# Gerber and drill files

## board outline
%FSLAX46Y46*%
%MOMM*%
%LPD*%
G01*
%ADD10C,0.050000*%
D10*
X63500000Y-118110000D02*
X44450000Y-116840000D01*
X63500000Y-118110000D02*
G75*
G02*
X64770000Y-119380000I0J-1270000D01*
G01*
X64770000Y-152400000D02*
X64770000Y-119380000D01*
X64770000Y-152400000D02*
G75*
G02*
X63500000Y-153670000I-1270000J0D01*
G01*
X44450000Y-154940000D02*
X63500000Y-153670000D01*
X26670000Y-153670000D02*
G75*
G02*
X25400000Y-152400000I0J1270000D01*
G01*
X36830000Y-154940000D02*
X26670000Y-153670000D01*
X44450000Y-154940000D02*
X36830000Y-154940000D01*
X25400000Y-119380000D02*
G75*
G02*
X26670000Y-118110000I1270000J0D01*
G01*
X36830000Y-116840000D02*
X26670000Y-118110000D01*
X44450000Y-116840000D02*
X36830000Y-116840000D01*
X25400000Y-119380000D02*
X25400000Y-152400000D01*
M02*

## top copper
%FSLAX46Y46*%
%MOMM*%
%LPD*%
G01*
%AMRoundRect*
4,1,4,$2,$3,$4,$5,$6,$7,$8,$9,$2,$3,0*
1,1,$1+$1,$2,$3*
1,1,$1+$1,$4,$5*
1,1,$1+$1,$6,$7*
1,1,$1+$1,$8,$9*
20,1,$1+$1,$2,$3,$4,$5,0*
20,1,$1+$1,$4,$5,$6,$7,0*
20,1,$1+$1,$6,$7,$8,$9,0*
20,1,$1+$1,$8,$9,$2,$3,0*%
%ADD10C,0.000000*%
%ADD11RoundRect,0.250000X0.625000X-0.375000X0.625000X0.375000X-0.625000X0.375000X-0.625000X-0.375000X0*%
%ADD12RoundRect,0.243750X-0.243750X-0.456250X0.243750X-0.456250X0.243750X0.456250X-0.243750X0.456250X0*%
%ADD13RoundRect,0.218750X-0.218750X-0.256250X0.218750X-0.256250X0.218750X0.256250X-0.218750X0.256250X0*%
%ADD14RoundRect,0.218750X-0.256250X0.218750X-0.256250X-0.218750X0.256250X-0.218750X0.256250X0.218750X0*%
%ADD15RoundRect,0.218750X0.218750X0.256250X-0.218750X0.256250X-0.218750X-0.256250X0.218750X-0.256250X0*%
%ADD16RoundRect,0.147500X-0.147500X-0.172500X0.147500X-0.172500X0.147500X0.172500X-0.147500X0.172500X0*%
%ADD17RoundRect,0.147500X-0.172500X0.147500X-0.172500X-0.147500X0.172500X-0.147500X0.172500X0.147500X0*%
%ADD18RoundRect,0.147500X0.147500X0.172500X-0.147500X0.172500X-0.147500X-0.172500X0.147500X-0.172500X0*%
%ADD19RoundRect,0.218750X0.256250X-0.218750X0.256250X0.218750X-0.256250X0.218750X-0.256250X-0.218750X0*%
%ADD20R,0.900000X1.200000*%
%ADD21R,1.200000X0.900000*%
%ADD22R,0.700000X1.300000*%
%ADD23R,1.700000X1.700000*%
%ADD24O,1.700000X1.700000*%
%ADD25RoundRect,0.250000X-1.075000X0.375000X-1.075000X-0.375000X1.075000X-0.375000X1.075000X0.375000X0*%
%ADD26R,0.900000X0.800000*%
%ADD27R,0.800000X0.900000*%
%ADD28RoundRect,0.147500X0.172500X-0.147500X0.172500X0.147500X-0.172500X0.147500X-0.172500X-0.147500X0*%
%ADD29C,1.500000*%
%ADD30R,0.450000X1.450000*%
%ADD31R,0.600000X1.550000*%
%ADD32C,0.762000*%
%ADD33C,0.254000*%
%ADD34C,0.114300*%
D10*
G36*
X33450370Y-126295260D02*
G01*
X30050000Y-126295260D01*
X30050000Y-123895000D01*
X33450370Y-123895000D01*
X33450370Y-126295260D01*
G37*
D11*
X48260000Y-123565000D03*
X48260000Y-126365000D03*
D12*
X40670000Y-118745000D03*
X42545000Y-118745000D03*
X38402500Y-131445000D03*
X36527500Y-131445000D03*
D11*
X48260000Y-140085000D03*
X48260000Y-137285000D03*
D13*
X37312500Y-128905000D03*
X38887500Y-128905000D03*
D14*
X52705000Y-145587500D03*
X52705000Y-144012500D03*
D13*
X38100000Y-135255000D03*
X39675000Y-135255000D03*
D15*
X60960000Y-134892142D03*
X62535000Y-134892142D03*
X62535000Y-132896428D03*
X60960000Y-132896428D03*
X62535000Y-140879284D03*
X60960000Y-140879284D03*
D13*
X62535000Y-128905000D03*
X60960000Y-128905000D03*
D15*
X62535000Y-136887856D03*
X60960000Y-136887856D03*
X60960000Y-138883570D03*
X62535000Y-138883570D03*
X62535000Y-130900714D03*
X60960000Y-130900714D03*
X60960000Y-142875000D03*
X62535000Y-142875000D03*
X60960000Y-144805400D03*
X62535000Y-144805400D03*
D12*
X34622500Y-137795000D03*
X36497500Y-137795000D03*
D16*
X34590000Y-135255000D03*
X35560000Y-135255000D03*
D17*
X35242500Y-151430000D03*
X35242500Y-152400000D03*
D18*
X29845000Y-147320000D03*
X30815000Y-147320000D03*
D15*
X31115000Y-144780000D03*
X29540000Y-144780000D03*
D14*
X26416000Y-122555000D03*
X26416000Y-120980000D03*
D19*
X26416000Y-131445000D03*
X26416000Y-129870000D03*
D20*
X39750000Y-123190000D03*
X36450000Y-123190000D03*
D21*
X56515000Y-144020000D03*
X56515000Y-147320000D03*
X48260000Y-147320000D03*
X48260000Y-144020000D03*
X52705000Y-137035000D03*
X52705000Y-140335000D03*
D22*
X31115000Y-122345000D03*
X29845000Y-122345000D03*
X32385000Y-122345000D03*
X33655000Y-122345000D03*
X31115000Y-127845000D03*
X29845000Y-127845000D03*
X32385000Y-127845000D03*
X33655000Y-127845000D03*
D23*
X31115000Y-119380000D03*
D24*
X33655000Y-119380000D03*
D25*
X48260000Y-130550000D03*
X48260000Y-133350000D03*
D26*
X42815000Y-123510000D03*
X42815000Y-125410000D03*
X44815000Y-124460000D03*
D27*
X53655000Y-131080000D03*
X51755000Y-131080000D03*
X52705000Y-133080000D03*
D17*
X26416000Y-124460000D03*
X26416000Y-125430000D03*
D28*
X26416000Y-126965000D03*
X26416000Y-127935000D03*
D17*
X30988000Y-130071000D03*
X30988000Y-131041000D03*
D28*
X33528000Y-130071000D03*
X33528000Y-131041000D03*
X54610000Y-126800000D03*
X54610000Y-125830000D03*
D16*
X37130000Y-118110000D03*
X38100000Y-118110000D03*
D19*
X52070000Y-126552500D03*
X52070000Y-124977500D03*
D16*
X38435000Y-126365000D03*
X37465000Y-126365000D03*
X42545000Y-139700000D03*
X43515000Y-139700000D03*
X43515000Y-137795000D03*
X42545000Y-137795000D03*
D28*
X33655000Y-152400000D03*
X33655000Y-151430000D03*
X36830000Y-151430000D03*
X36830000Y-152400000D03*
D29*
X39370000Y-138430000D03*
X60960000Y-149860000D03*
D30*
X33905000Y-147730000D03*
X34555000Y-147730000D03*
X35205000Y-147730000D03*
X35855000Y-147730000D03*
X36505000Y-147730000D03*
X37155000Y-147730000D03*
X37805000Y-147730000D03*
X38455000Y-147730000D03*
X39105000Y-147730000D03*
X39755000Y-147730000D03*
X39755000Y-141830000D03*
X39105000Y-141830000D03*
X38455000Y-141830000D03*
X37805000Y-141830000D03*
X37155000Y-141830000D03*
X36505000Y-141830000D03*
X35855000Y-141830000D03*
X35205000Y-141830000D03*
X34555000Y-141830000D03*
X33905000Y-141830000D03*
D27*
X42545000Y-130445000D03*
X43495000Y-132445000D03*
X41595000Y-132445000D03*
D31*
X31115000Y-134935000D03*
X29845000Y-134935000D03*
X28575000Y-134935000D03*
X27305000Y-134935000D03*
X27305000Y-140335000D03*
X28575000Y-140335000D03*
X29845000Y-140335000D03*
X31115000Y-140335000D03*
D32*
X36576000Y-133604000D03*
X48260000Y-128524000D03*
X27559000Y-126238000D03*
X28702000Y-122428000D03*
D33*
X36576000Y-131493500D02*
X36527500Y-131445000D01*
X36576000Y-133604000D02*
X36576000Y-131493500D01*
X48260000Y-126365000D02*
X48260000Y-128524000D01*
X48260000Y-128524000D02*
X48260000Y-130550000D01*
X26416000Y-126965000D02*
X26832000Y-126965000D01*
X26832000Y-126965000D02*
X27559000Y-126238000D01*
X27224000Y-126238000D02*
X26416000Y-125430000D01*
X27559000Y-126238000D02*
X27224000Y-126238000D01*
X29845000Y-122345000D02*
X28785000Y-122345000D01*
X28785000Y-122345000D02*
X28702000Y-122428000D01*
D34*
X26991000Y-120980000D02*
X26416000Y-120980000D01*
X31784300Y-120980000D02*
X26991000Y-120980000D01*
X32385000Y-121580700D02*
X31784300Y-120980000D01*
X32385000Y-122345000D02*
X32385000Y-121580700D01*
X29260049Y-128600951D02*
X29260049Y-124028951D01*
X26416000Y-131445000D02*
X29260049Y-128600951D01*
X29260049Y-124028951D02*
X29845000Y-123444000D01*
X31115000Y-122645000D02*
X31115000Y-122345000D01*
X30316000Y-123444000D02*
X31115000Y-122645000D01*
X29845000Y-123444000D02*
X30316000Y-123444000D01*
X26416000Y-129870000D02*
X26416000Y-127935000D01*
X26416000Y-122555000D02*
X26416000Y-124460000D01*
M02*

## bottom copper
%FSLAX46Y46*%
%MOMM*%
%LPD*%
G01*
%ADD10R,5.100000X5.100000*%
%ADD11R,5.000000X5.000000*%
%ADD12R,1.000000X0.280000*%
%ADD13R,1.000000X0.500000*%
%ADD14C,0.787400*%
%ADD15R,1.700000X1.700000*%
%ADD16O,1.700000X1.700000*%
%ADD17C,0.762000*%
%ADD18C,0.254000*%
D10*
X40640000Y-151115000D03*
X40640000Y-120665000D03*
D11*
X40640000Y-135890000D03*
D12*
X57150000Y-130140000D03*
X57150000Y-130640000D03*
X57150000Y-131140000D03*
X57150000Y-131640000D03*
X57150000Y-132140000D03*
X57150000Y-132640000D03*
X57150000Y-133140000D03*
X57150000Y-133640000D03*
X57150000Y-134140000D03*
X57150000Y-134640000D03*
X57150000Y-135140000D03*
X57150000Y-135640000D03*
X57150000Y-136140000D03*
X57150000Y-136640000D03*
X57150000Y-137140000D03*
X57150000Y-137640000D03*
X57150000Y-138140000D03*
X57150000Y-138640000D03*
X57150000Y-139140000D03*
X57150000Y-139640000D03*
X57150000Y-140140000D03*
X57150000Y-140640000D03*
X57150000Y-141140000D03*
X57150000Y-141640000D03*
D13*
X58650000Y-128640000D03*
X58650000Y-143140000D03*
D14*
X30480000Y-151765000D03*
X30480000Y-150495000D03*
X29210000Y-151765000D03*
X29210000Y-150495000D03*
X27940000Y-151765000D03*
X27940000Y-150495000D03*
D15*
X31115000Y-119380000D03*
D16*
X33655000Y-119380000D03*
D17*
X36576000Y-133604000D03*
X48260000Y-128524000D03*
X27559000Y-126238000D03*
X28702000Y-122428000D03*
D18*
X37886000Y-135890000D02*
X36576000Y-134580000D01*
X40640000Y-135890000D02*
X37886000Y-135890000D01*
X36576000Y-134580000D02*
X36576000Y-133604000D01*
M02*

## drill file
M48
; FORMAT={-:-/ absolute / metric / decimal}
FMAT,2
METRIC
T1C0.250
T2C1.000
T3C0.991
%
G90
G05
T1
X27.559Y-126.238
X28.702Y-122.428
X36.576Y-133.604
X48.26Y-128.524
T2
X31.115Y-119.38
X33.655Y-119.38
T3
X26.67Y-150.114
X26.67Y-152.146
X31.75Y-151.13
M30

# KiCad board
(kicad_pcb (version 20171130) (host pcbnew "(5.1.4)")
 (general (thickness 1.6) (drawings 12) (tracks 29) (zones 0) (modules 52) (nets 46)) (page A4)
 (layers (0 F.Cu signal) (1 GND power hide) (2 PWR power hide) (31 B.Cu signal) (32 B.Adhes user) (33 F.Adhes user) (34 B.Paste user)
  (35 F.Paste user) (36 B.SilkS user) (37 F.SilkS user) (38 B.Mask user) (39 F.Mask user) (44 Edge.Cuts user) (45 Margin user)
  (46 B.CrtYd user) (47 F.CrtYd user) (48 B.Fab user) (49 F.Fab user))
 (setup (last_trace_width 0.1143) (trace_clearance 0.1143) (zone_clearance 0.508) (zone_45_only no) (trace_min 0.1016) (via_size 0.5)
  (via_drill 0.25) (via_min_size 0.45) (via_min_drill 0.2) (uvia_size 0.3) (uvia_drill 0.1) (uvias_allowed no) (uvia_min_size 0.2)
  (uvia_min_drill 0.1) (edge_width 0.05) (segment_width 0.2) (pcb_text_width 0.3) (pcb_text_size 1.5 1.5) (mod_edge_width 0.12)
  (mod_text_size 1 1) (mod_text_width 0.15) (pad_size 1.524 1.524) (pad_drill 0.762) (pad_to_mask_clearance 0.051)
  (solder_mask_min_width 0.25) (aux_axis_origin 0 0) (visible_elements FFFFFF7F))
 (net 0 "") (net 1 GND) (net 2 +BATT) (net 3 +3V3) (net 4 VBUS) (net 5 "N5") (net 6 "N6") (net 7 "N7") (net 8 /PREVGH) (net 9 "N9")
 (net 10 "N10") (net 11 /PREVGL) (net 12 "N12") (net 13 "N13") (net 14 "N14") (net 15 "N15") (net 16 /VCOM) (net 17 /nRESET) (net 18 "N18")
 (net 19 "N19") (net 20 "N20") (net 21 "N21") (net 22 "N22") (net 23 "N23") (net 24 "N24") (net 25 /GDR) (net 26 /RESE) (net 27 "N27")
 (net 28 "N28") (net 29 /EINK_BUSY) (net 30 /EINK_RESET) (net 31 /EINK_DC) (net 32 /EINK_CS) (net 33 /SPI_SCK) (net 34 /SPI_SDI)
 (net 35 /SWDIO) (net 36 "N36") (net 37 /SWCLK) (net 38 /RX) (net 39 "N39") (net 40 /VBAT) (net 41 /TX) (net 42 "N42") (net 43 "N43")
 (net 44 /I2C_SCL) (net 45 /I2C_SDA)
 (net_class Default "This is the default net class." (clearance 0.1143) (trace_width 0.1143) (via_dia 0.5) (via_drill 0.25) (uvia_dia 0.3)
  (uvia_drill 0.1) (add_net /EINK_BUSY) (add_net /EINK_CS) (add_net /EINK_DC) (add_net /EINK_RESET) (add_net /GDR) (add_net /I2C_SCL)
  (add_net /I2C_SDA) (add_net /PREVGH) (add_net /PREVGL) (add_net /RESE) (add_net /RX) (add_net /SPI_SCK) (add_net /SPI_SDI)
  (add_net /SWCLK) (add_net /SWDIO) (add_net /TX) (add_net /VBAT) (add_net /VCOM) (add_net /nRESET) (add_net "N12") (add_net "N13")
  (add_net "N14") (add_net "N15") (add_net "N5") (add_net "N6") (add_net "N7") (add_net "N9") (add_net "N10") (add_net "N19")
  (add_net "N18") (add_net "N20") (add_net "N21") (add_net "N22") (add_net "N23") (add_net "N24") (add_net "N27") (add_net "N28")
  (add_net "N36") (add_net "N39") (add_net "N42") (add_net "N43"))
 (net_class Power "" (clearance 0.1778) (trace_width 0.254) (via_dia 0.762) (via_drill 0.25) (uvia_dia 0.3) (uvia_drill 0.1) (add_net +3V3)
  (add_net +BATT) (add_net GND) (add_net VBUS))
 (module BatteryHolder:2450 (layer B.Cu) (at 40.64 135.89)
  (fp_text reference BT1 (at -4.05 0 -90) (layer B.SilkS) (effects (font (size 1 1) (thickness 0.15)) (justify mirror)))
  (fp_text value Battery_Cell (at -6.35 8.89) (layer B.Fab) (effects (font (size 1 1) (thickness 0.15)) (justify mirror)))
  (pad 2 smd rect (at 0 15.225) (size 5.1 5.1) (layers B.Cu B.Paste B.Mask) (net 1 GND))
  (pad 2 smd rect (at 0 -15.225) (size 5.1 5.1) (layers B.Cu B.Paste B.Mask) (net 1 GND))
  (pad 1 smd rect (at 0 0) (size 5 5) (layers B.Cu B.Paste B.Mask) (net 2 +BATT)))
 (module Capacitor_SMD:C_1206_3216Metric (layer F.Cu) (at 48.26 124.965 90)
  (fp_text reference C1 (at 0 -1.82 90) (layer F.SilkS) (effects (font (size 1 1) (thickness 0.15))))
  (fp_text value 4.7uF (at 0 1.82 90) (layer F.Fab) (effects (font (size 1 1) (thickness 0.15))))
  (pad 2 smd roundrect (at 1.4 0 90) (size 1.25 1.75) (layers F.Cu F.Paste F.Mask) (roundrect_rratio 0.2) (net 1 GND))
  (pad 1 smd roundrect (at -1.4 0 90) (size 1.25 1.75) (layers F.Cu F.Paste F.Mask) (roundrect_rratio 0.2) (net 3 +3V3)))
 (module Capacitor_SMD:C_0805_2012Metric (layer F.Cu) (at 41.6075 118.745)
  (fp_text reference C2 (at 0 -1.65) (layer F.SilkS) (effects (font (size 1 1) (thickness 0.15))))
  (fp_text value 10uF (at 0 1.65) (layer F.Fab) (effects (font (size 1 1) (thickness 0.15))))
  (pad 1 smd roundrect (at -0.9375 0) (size 0.975 1.4) (layers F.Cu F.Paste F.Mask) (roundrect_rratio 0.25) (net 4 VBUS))
  (pad 2 smd roundrect (at 0.9375 0) (size 0.975 1.4) (layers F.Cu F.Paste F.Mask) (roundrect_rratio 0.25) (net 1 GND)))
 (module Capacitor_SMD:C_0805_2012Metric (layer F.Cu) (at 37.465 131.445)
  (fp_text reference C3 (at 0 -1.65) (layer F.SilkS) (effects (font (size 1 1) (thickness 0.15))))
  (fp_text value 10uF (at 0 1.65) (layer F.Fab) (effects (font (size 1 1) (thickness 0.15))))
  (pad 2 smd roundrect (at 0.9375 0) (size 0.975 1.4) (layers F.Cu F.Paste F.Mask) (roundrect_rratio 0.25) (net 1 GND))
  (pad 1 smd roundrect (at -0.9375 0) (size 0.975 1.4) (layers F.Cu F.Paste F.Mask) (roundrect_rratio 0.25) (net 2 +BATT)))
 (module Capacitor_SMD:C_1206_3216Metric (layer F.Cu) (at 48.26 138.685 90)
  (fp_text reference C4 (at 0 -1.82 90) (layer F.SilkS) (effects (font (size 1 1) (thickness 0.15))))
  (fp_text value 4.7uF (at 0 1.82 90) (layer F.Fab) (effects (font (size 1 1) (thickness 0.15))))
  (pad 1 smd roundrect (at -1.4 0 90) (size 1.25 1.75) (layers F.Cu F.Paste F.Mask) (roundrect_rratio 0.2) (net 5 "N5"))
  (pad 2 smd roundrect (at 1.4 0 90) (size 1.25 1.75) (layers F.Cu F.Paste F.Mask) (roundrect_rratio 0.2) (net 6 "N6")))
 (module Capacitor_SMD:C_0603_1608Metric (layer F.Cu) (at 38.1 128.905)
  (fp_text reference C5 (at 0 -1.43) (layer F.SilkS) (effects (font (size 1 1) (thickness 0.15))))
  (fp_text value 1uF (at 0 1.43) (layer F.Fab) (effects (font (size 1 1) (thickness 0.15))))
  (pad 1 smd roundrect (at -0.7875 0) (size 0.875 0.95) (layers F.Cu F.Paste F.Mask) (roundrect_rratio 0.25) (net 1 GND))
  (pad 2 smd roundrect (at 0.7875 0) (size 0.875 0.95) (layers F.Cu F.Paste F.Mask) (roundrect_rratio 0.25) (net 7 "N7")))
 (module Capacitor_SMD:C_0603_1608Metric (layer F.Cu) (at 52.705 144.8 270)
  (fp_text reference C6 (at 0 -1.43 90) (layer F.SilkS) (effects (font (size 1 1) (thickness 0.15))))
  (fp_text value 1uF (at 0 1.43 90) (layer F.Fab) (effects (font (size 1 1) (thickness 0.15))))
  (pad 2 smd roundrect (at 0.7875 0 270) (size 0.875 0.95) (layers F.Cu F.Paste F.Mask) (roundrect_rratio 0.25) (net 1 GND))
  (pad 1 smd roundrect (at -0.7875 0 270) (size 0.875 0.95) (layers F.Cu F.Paste F.Mask) (roundrect_rratio 0.25) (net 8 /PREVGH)))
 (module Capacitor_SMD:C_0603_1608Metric (layer F.Cu) (at 38.8875 135.255)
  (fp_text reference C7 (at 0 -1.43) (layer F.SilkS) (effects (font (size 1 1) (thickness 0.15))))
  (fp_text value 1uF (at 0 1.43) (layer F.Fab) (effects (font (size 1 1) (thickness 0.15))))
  (pad 1 smd roundrect (at -0.7875 0) (size 0.875 0.95) (layers F.Cu F.Paste F.Mask) (roundrect_rratio 0.25) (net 1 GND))
  (pad 2 smd roundrect (at 0.7875 0) (size 0.875 0.95) (layers F.Cu F.Paste F.Mask) (roundrect_rratio 0.25) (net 3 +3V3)))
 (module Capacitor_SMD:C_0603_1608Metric (layer F.Cu) (at 61.7475 134.892142 180)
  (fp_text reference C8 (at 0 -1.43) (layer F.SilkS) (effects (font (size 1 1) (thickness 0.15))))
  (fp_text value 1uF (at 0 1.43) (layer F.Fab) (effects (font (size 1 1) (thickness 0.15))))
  (pad 2 smd roundrect (at 0.7875 0 180) (size 0.875 0.95) (layers F.Cu F.Paste F.Mask) (roundrect_rratio 0.25) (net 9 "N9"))
  (pad 1 smd roundrect (at -0.7875 0 180) (size 0.875 0.95) (layers F.Cu F.Paste F.Mask) (roundrect_rratio 0.25) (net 1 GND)))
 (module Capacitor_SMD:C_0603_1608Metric (layer F.Cu) (at 61.7475 132.896428 180)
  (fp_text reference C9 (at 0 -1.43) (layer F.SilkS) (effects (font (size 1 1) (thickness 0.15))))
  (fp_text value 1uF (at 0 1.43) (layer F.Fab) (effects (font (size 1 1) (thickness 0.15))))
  (pad 1 smd roundrect (at -0.7875 0 180) (size 0.875 0.95) (layers F.Cu F.Paste F.Mask) (roundrect_rratio 0.25) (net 1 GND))
  (pad 2 smd roundrect (at 0.7875 0 180) (size 0.875 0.95) (layers F.Cu F.Paste F.Mask) (roundrect_rratio 0.25) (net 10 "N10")))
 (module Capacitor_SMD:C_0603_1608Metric (layer F.Cu) (at 61.7475 140.879284 180)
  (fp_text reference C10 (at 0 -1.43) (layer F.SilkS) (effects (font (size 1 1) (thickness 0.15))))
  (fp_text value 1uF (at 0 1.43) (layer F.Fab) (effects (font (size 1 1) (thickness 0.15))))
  (pad 1 smd roundrect (at -0.7875 0 180) (size 0.875 0.95) (layers F.Cu F.Paste F.Mask) (roundrect_rratio 0.25) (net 1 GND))
  (pad 2 smd roundrect (at 0.7875 0 180) (size 0.875 0.95) (layers F.Cu F.Paste F.Mask) (roundrect_rratio 0.25) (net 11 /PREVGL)))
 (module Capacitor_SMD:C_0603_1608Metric (layer F.Cu) (at 61.7475 128.905)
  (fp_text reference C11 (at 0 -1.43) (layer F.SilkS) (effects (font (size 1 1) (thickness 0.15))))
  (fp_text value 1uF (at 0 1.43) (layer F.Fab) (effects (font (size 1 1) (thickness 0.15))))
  (pad 2 smd roundrect (at 0.7875 0) (size 0.875 0.95) (layers F.Cu F.Paste F.Mask) (roundrect_rratio 0.25) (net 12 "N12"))
  (pad 1 smd roundrect (at -0.7875 0) (size 0.875 0.95) (layers F.Cu F.Paste F.Mask) (roundrect_rratio 0.25) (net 1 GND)))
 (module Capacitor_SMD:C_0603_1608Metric (layer F.Cu) (at 61.7475 136.887856 180)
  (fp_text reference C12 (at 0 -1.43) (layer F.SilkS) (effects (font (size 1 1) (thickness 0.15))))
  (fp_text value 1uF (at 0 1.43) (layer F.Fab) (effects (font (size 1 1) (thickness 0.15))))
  (pad 1 smd roundrect (at -0.7875 0 180) (size 0.875 0.95) (layers F.Cu F.Paste F.Mask) (roundrect_rratio 0.25) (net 1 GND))
  (pad 2 smd roundrect (at 0.7875 0 180) (size 0.875 0.95) (layers F.Cu F.Paste F.Mask) (roundrect_rratio 0.25) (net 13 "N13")))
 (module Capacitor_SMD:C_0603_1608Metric (layer F.Cu) (at 61.7475 138.88357 180)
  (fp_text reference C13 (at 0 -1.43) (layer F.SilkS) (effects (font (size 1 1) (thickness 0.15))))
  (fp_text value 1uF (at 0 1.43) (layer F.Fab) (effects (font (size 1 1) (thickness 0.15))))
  (pad 2 smd roundrect (at 0.7875 0 180) (size 0.875 0.95) (layers F.Cu F.Paste F.Mask) (roundrect_rratio 0.25) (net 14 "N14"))
  (pad 1 smd roundrect (at -0.7875 0 180) (size 0.875 0.95) (layers F.Cu F.Paste F.Mask) (roundrect_rratio 0.25) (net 1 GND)))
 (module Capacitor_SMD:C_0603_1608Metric (layer F.Cu) (at 61.7475 130.900714 180)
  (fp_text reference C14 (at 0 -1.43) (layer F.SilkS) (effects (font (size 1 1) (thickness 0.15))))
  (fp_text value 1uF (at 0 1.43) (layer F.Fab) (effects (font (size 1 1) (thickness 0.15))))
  (pad 1 smd roundrect (at -0.7875 0 180) (size 0.875 0.95) (layers F.Cu F.Paste F.Mask) (roundrect_rratio 0.25) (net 1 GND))
  (pad 2 smd roundrect (at 0.7875 0 180) (size 0.875 0.95) (layers F.Cu F.Paste F.Mask) (roundrect_rratio 0.25) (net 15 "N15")))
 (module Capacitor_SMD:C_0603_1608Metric (layer F.Cu) (at 61.7475 142.875 180)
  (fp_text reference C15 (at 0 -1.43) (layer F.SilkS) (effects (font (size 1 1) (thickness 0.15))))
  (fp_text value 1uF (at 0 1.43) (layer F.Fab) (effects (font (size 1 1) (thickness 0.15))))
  (pad 2 smd roundrect (at 0.7875 0 180) (size 0.875 0.95) (layers F.Cu F.Paste F.Mask) (roundrect_rratio 0.25) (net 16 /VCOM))
  (pad 1 smd roundrect (at -0.7875 0 180) (size 0.875 0.95) (layers F.Cu F.Paste F.Mask) (roundrect_rratio 0.25) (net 1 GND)))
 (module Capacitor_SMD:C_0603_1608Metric (layer F.Cu) (at 61.7475 144.8054 180)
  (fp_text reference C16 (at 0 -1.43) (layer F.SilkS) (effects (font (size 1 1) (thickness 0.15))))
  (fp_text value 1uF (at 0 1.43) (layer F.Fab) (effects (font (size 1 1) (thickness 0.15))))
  (pad 2 smd roundrect (at 0.7875 0 180) (size 0.875 0.95) (layers F.Cu F.Paste F.Mask) (roundrect_rratio 0.25) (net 3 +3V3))
  (pad 1 smd roundrect (at -0.7875 0 180) (size 0.875 0.95) (layers F.Cu F.Paste F.Mask) (roundrect_rratio 0.25) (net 1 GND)))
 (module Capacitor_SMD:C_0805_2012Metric (layer F.Cu) (at 35.56 137.795)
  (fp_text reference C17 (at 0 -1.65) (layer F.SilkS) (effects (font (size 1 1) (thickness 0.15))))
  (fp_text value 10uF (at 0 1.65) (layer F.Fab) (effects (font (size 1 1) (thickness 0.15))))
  (pad 1 smd roundrect (at -0.9375 0) (size 0.975 1.4) (layers F.Cu F.Paste F.Mask) (roundrect_rratio 0.25) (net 3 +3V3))
  (pad 2 smd roundrect (at 0.9375 0) (size 0.975 1.4) (layers F.Cu F.Paste F.Mask) (roundrect_rratio 0.25) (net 1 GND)))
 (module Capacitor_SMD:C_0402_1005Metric (layer F.Cu) (at 35.075 135.255)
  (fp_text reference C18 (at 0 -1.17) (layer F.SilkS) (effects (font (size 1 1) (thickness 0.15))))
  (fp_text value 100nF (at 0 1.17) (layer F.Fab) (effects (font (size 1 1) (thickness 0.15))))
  (pad 1 smd roundrect (at -0.485 0) (size 0.59 0.64) (layers F.Cu F.Paste F.Mask) (roundrect_rratio 0.25) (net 3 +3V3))
  (pad 2 smd roundrect (at 0.485 0) (size 0.59 0.64) (layers F.Cu F.Paste F.Mask) (roundrect_rratio 0.25) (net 1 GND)))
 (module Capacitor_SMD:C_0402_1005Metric (layer F.Cu) (at 35.2425 151.915 270)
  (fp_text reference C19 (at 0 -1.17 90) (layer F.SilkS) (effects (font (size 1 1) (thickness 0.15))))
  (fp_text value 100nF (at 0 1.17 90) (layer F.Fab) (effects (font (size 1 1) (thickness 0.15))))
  (pad 1 smd roundrect (at -0.485 0 270) (size 0.59 0.64) (layers F.Cu F.Paste F.Mask) (roundrect_rratio 0.25) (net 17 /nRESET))
  (pad 2 smd roundrect (at 0.485 0 270) (size 0.59 0.64) (layers F.Cu F.Paste F.Mask) (roundrect_rratio 0.25) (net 1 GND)))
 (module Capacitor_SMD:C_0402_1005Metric (layer F.Cu) (at 30.33 147.32 180)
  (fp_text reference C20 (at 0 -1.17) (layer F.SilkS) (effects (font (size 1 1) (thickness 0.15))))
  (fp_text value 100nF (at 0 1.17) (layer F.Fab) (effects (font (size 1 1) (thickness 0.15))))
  (pad 2 smd roundrect (at 0.485 0 180) (size 0.59 0.64) (layers F.Cu F.Paste F.Mask) (roundrect_rratio 0.25) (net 1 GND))
  (pad 1 smd roundrect (at -0.485 0 180) (size 0.59 0.64) (layers F.Cu F.Paste F.Mask) (roundrect_rratio 0.25) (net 3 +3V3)))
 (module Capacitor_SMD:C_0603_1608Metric (layer F.Cu) (at 30.3275 144.78 180)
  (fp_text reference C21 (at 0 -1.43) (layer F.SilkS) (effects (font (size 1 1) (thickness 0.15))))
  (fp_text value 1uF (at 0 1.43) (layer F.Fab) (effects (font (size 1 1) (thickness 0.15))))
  (pad 1 smd roundrect (at -0.7875 0 180) (size 0.875 0.95) (layers F.Cu F.Paste F.Mask) (roundrect_rratio 0.25) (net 3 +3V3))
  (pad 2 smd roundrect (at 0.7875 0 180) (size 0.875 0.95) (layers F.Cu F.Paste F.Mask) (roundrect_rratio 0.25) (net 1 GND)))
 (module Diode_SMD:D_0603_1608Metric (layer F.Cu) (at 26.416 121.7675 270)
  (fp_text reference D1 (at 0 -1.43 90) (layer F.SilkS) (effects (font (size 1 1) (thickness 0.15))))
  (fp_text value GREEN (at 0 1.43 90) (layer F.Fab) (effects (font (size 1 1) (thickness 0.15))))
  (pad 2 smd roundrect (at 0.7875 0 270) (size 0.875 0.95) (layers F.Cu F.Paste F.Mask) (roundrect_rratio 0.25) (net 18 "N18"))
  (pad 1 smd roundrect (at -0.7875 0 270) (size 0.875 0.95) (layers F.Cu F.Paste F.Mask) (roundrect_rratio 0.25) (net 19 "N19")))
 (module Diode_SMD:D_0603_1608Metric (layer F.Cu) (at 26.416 130.6575 90)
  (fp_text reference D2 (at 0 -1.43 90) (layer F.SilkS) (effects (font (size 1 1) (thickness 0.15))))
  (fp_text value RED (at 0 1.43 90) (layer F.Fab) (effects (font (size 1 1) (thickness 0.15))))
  (pad 1 smd roundrect (at -0.7875 0 90) (size 0.875 0.95) (layers F.Cu F.Paste F.Mask) (roundrect_rratio 0.25) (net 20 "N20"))
  (pad 2 smd roundrect (at 0.7875 0 90) (size 0.875 0.95) (layers F.Cu F.Paste F.Mask) (roundrect_rratio 0.25) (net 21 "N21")))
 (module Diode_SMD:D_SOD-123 (layer F.Cu) (at 38.1 123.19 180)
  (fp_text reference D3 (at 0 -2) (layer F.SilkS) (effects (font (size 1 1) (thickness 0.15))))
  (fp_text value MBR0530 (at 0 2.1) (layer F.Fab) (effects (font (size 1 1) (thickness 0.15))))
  (pad 1 smd rect (at -1.65 0 180) (size 0.9 1.2) (layers F.Cu F.Paste F.Mask) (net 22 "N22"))
  (pad 2 smd rect (at 1.65 0 180) (size 0.9 1.2) (layers F.Cu F.Paste F.Mask) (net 4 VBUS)))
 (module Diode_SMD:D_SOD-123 (layer F.Cu) (at 56.515 145.67 90)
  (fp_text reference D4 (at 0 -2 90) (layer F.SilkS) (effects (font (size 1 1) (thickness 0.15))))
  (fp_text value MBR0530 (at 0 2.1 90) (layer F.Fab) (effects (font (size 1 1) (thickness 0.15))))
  (pad 2 smd rect (at 1.65 0 90) (size 0.9 1.2) (layers F.Cu F.Paste F.Mask) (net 11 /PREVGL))
  (pad 1 smd rect (at -1.65 0 90) (size 0.9 1.2) (layers F.Cu F.Paste F.Mask) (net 5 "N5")))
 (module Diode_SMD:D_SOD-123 (layer F.Cu) (at 48.26 145.67 90)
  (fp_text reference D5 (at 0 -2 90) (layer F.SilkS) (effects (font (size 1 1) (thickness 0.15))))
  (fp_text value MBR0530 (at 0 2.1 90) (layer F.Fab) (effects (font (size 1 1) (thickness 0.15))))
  (pad 1 smd rect (at -1.65 0 90) (size 0.9 1.2) (layers F.Cu F.Paste F.Mask) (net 1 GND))
  (pad 2 smd rect (at 1.65 0 90) (size 0.9 1.2) (layers F.Cu F.Paste F.Mask) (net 5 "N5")))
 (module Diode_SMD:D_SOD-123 (layer F.Cu) (at 52.705 138.685 90)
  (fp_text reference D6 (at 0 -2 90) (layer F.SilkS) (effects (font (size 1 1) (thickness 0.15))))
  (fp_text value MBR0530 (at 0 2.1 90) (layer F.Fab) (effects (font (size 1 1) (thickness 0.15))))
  (pad 2 smd rect (at 1.65 0 90) (size 0.9 1.2) (layers F.Cu F.Paste F.Mask) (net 6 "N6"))
  (pad 1 smd rect (at -1.65 0 90) (size 0.9 1.2) (layers F.Cu F.Paste F.Mask) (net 8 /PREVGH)))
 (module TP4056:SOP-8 (layer F.Cu) (at 31.75 125.095 90)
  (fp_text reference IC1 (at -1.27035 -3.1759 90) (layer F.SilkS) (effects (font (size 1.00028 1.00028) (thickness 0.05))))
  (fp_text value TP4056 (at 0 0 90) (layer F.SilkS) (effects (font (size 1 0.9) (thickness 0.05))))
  (fp_poly (pts (xy -1.20026 -1.7) (xy 1.2 -1.7) (xy 1.2 1.70037) (xy -1.20026 1.70037)) (layer F.Cu) (width 0))
  (pad 7 smd rect (at 2.75 -0.635 90) (size 1.3 0.7) (layers F.Cu F.Paste F.Mask) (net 20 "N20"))
  (pad 8 smd rect (at 2.75 -1.905 90) (size 1.3 0.7) (layers F.Cu F.Paste F.Mask) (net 4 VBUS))
  (pad 6 smd rect (at 2.75 0.635 90) (size 1.3 0.7) (layers F.Cu F.Paste F.Mask) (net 19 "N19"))
  (pad 5 smd rect (at 2.75 1.905 90) (size 1.3 0.7) (layers F.Cu F.Paste F.Mask) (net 2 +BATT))
  (pad 2 smd rect (at -2.75 -0.635 90) (size 1.3 0.7) (layers F.Cu F.Paste F.Mask) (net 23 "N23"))
  (pad 1 smd rect (at -2.75 -1.905 90) (size 1.3 0.7) (layers F.Cu F.Paste F.Mask) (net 1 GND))
  (pad 3 smd rect (at -2.75 0.635 90) (size 1.3 0.7) (layers F.Cu F.Paste F.Mask) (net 1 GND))
  (pad 4 smd rect (at -2.75 1.905 90) (size 1.3 0.7) (layers F.Cu F.Paste F.Mask) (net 4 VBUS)))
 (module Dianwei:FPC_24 (layer B.Cu) (at 57.15 135.89 270)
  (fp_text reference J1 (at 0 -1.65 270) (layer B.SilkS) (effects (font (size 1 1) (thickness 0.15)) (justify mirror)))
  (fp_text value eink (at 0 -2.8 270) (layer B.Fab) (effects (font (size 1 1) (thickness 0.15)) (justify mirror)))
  (pad 1 smd rect (at -5.75 0 270) (size 0.28 1) (layers B.Cu B.Paste B.Mask) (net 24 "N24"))
  (pad 2 smd rect (at -5.25 0 270) (size 0.28 1) (layers B.Cu B.Paste B.Mask) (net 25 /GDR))
  (pad 3 smd rect (at -4.75 0 270) (size 0.28 1) (layers B.Cu B.Paste B.Mask) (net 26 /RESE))
  (pad 4 smd rect (at -4.25 0 270) (size 0.28 1) (layers B.Cu B.Paste B.Mask) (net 12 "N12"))
  (pad 5 smd rect (at -3.75 0 270) (size 0.28 1) (layers B.Cu B.Paste B.Mask) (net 15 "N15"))
  (pad 6 smd rect (at -3.25 0 270) (size 0.28 1) (layers B.Cu B.Paste B.Mask) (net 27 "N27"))
  (pad 7 smd rect (at -2.75 0 270) (size 0.28 1) (layers B.Cu B.Paste B.Mask) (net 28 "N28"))
  (pad 8 smd rect (at -2.25 0 270) (size 0.28 1) (layers B.Cu B.Paste B.Mask) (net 1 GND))
  (pad 9 smd rect (at -1.75 0 270) (size 0.28 1) (layers B.Cu B.Paste B.Mask) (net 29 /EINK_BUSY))
  (pad 10 smd rect (at -1.25 0 270) (size 0.28 1) (layers B.Cu B.Paste B.Mask) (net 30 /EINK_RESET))
  (pad 11 smd rect (at -0.75 0 270) (size 0.28 1) (layers B.Cu B.Paste B.Mask) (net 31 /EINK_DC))
  (pad 12 smd rect (at -0.25 0 270) (size 0.28 1) (layers B.Cu B.Paste B.Mask) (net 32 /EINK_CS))
  (pad 13 smd rect (at 0.25 0 270) (size 0.28 1) (layers B.Cu B.Paste B.Mask) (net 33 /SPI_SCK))
  (pad 14 smd rect (at 0.75 0 270) (size 0.28 1) (layers B.Cu B.Paste B.Mask) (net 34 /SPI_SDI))
  (pad 15 smd rect (at 1.25 0 270) (size 0.28 1) (layers B.Cu B.Paste B.Mask) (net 3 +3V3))
  (pad 16 smd rect (at 1.75 0 270) (size 0.28 1) (layers B.Cu B.Paste B.Mask) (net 3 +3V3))
  (pad 17 smd rect (at 2.25 0 270) (size 0.28 1) (layers B.Cu B.Paste B.Mask) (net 1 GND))
  (pad 18 smd rect (at 2.75 0 270) (size 0.28 1) (layers B.Cu B.Paste B.Mask) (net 10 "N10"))
  (pad 19 smd rect (at 3.25 0 270) (size 0.28 1) (layers B.Cu B.Paste B.Mask) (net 9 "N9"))
  (pad 20 smd rect (at 3.75 0 270) (size 0.28 1) (layers B.Cu B.Paste B.Mask) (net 13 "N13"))
  (pad 21 smd rect (at 4.25 0 270) (size 0.28 1) (layers B.Cu B.Paste B.Mask) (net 8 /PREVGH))
  (pad 22 smd rect (at 4.75 0 270) (size 0.28 1) (layers B.Cu B.Paste B.Mask) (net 14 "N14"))
  (pad 23 smd rect (at 5.25 0 270) (size 0.28 1) (layers B.Cu B.Paste B.Mask) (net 11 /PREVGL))
  (pad 24 smd rect (at 5.75 0 270) (size 0.28 1) (layers B.Cu B.Paste B.Mask) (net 16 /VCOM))
  (pad 0 smd rect (at -7.25 -1.5 270) (size 0.5 1) (layers B.Cu B.Paste B.Mask))
  (pad 0 smd rect (at 7.25 -1.5 270) (size 0.5 1) (layers B.Cu B.Paste B.Mask)))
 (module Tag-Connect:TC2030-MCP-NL (layer B.Cu) (at 29.21 151.13 180)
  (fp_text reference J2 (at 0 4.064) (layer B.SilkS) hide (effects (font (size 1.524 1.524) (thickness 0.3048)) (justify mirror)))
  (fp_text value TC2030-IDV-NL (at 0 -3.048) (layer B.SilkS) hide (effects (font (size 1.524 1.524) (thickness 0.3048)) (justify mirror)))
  (pad 1 connect circle (at -1.27 -0.635 180) (size 0.7874 0.7874) (layers B.Cu B.Mask) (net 3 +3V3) (clearance 0.4826))
  (pad 2 connect circle (at -1.27 0.635 180) (size 0.7874 0.7874) (layers B.Cu B.Mask) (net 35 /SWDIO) (clearance 0.4826))
  (pad 3 connect circle (at 0 -0.635 180) (size 0.7874 0.7874) (layers B.Cu B.Mask) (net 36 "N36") (clearance 0.4826))
  (pad 4 connect circle (at 0 0.635 180) (size 0.7874 0.7874) (layers B.Cu B.Mask) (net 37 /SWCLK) (clearance 0.4826))
  (pad 5 connect circle (at 1.27 -0.635 180) (size 0.7874 0.7874) (layers B.Cu B.Mask) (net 1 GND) (clearance 0.4318))
  (pad 6 connect circle (at 1.27 0.635 180) (size 0.7874 0.7874) (layers B.Cu B.Mask) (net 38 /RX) (clearance 0.4318))
  (pad "" np_thru_hole circle (at -2.54 0 180) (size 0.9906 0.9906) (drill 0.9906) (layers *.Cu *.Mask B.SilkS))
  (pad "" np_thru_hole circle (at 2.54 1.016 180) (size 0.9906 0.9906) (drill 0.9906) (layers *.Cu *.Mask B.SilkS))
  (pad "" np_thru_hole circle (at 2.54 -1.016 180) (size 0.9906 0.9906) (drill 0.9906) (layers *.Cu *.Mask B.SilkS)))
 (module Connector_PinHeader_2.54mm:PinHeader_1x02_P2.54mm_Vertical (layer F.Cu) (at 31.115 119.38 90)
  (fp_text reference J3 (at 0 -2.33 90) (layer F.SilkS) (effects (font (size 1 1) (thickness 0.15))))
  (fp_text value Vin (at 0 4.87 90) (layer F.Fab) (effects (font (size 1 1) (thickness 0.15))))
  (pad 1 thru_hole rect (at 0 0 90) (size 1.7 1.7) (drill 1) (layers *.Cu *.Mask) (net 1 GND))
  (pad 2 thru_hole oval (at 0 2.54 90) (size 1.7 1.7) (drill 1) (layers *.Cu *.Mask) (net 4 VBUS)))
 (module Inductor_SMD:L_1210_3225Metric (layer F.Cu) (at 48.26 131.95 270)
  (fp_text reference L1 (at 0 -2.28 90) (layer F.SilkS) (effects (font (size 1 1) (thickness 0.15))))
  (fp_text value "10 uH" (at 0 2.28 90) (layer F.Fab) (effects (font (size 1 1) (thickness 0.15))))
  (pad 1 smd roundrect (at -1.4 0 270) (size 1.25 2.65) (layers F.Cu F.Paste F.Mask) (roundrect_rratio 0.2) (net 3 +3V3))
  (pad 2 smd roundrect (at 1.4 0 270) (size 1.25 2.65) (layers F.Cu F.Paste F.Mask) (roundrect_rratio 0.2) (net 6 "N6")))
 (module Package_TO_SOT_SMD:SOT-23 (layer F.Cu) (at 43.815 124.46)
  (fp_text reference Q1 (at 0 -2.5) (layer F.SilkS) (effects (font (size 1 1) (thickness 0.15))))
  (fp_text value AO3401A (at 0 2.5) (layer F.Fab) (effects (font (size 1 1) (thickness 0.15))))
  (pad 1 smd rect (at -1 -0.95) (size 0.9 0.8) (layers F.Cu F.Paste F.Mask) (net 4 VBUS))
  (pad 2 smd rect (at -1 0.95) (size 0.9 0.8) (layers F.Cu F.Paste F.Mask) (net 22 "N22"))
  (pad 3 smd rect (at 1 0) (size 0.9 0.8) (layers F.Cu F.Paste F.Mask) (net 2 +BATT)))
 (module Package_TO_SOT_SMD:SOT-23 (layer F.Cu) (at 52.705 132.08 270)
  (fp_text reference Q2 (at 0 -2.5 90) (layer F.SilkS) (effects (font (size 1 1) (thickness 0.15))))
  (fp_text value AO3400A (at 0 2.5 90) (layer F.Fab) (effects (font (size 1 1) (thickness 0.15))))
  (pad 1 smd rect (at -1 -0.95 270) (size 0.9 0.8) (layers F.Cu F.Paste F.Mask) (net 25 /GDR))
  (pad 2 smd rect (at -1 0.95 270) (size 0.9 0.8) (layers F.Cu F.Paste F.Mask) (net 26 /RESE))
  (pad 3 smd rect (at 1 0 270) (size 0.9 0.8) (layers F.Cu F.Paste F.Mask) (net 6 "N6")))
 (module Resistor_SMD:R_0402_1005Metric (layer F.Cu) (at 26.416 124.945 270)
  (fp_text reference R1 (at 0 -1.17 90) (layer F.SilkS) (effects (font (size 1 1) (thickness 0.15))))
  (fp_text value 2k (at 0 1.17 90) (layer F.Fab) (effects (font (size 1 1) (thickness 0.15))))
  (pad 1 smd roundrect (at -0.485 0 270) (size 0.59 0.64) (layers F.Cu F.Paste F.Mask) (roundrect_rratio 0.25) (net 18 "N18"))
  (pad 2 smd roundrect (at 0.485 0 270) (size 0.59 0.64) (layers F.Cu F.Paste F.Mask) (roundrect_rratio 0.25) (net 4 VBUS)))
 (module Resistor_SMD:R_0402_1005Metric (layer F.Cu) (at 26.416 127.45 90)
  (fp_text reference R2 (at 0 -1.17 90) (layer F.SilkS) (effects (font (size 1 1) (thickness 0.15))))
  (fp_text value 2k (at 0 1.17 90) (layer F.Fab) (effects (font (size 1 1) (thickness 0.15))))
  (pad 2 smd roundrect (at 0.485 0 90) (size 0.59 0.64) (layers F.Cu F.Paste F.Mask) (roundrect_rratio 0.25) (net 4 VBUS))
  (pad 1 smd roundrect (at -0.485 0 90) (size 0.59 0.64) (layers F.Cu F.Paste F.Mask) (roundrect_rratio 0.25) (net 21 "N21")))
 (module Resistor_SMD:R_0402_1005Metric (layer F.Cu) (at 30.988 130.556 270)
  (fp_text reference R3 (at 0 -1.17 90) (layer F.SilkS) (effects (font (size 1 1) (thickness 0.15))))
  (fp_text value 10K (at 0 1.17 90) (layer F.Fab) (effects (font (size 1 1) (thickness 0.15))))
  (pad 1 smd roundrect (at -0.485 0 270) (size 0.59 0.64) (layers F.Cu F.Paste F.Mask) (roundrect_rratio 0.25) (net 23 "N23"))
  (pad 2 smd roundrect (at 0.485 0 270) (size 0.59 0.64) (layers F.Cu F.Paste F.Mask) (roundrect_rratio 0.25) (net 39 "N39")))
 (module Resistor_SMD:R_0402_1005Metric (layer F.Cu) (at 33.528 130.556 90)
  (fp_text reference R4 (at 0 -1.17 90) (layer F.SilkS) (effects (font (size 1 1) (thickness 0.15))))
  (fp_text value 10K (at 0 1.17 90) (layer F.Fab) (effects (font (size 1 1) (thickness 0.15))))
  (pad 2 smd roundrect (at 0.485 0 90) (size 0.59 0.64) (layers F.Cu F.Paste F.Mask) (roundrect_rratio 0.25) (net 1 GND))
  (pad 1 smd roundrect (at -0.485 0 90) (size 0.59 0.64) (layers F.Cu F.Paste F.Mask) (roundrect_rratio 0.25) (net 39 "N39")))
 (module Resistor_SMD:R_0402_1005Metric (layer F.Cu) (at 54.61 126.315 90)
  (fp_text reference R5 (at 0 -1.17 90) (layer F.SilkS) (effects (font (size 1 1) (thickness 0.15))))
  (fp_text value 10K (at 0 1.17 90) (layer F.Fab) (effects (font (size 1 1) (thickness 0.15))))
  (pad 1 smd roundrect (at -0.485 0 90) (size 0.59 0.64) (layers F.Cu F.Paste F.Mask) (roundrect_rratio 0.25) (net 25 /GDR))
  (pad 2 smd roundrect (at 0.485 0 90) (size 0.59 0.64) (layers F.Cu F.Paste F.Mask) (roundrect_rratio 0.25) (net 1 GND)))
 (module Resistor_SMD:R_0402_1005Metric (layer F.Cu) (at 37.615 118.11)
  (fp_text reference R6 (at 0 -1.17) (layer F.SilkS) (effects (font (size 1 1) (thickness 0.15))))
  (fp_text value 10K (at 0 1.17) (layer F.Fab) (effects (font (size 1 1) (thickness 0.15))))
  (pad 1 smd roundrect (at -0.485 0) (size 0.59 0.64) (layers F.Cu F.Paste F.Mask) (roundrect_rratio 0.25) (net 4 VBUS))
  (pad 2 smd roundrect (at 0.485 0) (size 0.59 0.64) (layers F.Cu F.Paste F.Mask) (roundrect_rratio 0.25) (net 1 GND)))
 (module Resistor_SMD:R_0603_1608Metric (layer F.Cu) (at 52.07 125.765 90)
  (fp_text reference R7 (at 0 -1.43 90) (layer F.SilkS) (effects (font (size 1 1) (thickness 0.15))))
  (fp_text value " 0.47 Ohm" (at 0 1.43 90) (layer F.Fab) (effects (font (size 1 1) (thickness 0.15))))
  (pad 1 smd roundrect (at -0.7875 0 90) (size 0.875 0.95) (layers F.Cu F.Paste F.Mask) (roundrect_rratio 0.25) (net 26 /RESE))
  (pad 2 smd roundrect (at 0.7875 0 90) (size 0.875 0.95) (layers F.Cu F.Paste F.Mask) (roundrect_rratio 0.25) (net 1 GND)))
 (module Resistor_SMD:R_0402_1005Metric (layer F.Cu) (at 37.95 126.365)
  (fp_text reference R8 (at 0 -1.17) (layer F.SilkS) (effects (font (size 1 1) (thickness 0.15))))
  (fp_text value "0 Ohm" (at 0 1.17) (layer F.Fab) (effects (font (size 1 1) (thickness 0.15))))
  (pad 2 smd roundrect (at 0.485 0) (size 0.59 0.64) (layers F.Cu F.Paste F.Mask) (roundrect_rratio 0.25) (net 22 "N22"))
  (pad 1 smd roundrect (at -0.485 0) (size 0.59 0.64) (layers F.Cu F.Paste F.Mask) (roundrect_rratio 0.25) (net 7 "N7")))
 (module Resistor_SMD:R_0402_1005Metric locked (layer F.Cu) (at 43.03 139.7)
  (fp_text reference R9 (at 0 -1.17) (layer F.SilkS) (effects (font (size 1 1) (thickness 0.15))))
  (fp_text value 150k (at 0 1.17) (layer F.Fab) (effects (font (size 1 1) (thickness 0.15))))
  (pad 1 smd roundrect (at -0.485 0) (size 0.59 0.64) (layers F.Cu F.Paste F.Mask) (roundrect_rratio 0.25) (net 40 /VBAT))
  (pad 2 smd roundrect (at 0.485 0) (size 0.59 0.64) (layers F.Cu F.Paste F.Mask) (roundrect_rratio 0.25) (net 2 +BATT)))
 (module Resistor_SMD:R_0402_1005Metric (layer F.Cu) (at 43.03 137.795)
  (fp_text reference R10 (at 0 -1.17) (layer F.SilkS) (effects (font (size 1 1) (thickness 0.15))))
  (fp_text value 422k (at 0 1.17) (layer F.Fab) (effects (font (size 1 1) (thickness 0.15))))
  (pad 2 smd roundrect (at 0.485 0) (size 0.59 0.64) (layers F.Cu F.Paste F.Mask) (roundrect_rratio 0.25) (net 1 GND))
  (pad 1 smd roundrect (at -0.485 0) (size 0.59 0.64) (layers F.Cu F.Paste F.Mask) (roundrect_rratio 0.25) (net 40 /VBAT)))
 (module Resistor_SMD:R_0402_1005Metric (layer F.Cu) (at 33.655 151.915 90)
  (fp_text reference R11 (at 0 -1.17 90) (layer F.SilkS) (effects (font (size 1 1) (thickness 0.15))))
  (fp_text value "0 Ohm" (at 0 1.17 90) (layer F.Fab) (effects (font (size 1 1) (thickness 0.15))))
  (pad 1 smd roundrect (at -0.485 0 90) (size 0.59 0.64) (layers F.Cu F.Paste F.Mask) (roundrect_rratio 0.25) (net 36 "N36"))
  (pad 2 smd roundrect (at 0.485 0 90) (size 0.59 0.64) (layers F.Cu F.Paste F.Mask) (roundrect_rratio 0.25) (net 17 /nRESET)))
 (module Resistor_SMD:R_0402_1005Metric (layer F.Cu) (at 36.83 151.915 90)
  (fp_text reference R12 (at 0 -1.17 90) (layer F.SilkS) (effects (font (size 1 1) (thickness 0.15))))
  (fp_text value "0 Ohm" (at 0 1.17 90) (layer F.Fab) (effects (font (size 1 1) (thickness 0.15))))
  (pad 2 smd roundrect (at 0.485 0 90) (size 0.59 0.64) (layers F.Cu F.Paste F.Mask) (roundrect_rratio 0.25) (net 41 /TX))
  (pad 1 smd roundrect (at -0.485 0 90) (size 0.59 0.64) (layers F.Cu F.Paste F.Mask) (roundrect_rratio 0.25) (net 36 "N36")))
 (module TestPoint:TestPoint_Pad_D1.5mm (layer F.Cu) (at 39.37 138.43)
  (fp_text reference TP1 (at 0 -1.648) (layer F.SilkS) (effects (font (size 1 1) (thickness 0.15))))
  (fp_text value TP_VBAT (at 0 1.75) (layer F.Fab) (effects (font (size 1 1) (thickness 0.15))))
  (pad 1 smd circle (at 0 0) (size 1.5 1.5) (layers F.Cu F.Mask) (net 40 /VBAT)))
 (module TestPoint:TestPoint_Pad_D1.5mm (layer F.Cu) (at 60.96 149.86)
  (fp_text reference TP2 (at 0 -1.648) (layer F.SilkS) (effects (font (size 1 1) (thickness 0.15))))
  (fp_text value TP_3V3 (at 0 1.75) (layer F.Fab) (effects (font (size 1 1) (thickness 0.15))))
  (pad 1 smd circle (at 0 0) (size 1.5 1.5) (layers F.Cu F.Mask) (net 3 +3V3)))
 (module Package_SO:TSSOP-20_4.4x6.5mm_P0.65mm (layer F.Cu) (at 36.83 144.78 90)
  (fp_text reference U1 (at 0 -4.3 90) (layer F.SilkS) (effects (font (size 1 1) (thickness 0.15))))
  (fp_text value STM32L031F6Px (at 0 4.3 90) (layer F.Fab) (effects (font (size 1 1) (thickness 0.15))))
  (pad 1 smd rect (at -2.95 -2.925 90) (size 1.45 0.45) (layers F.Cu F.Paste F.Mask) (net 1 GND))
  (pad 2 smd rect (at -2.95 -2.275 90) (size 1.45 0.45) (layers F.Cu F.Paste F.Mask) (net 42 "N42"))
  (pad 3 smd rect (at -2.95 -1.625 90) (size 1.45 0.45) (layers F.Cu F.Paste F.Mask) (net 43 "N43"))
  (pad 4 smd rect (at -2.95 -0.975 90) (size 1.45 0.45) (layers F.Cu F.Paste F.Mask) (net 17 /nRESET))
  (pad 5 smd rect (at -2.95 -0.325 90) (size 1.45 0.45) (layers F.Cu F.Paste F.Mask) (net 3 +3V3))
  (pad 6 smd rect (at -2.95 0.325 90) (size 1.45 0.45) (layers F.Cu F.Paste F.Mask) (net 32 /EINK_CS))
  (pad 7 smd rect (at -2.95 0.975 90) (size 1.45 0.45) (layers F.Cu F.Paste F.Mask) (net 30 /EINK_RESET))
  (pad 8 smd rect (at -2.95 1.625 90) (size 1.45 0.45) (layers F.Cu F.Paste F.Mask) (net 41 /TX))
  (pad 9 smd rect (at -2.95 2.275 90) (size 1.45 0.45) (layers F.Cu F.Paste F.Mask) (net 38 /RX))
  (pad 10 smd rect (at -2.95 2.925 90) (size 1.45 0.45) (layers F.Cu F.Paste F.Mask) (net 31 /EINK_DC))
  (pad 11 smd rect (at 2.95 2.925 90) (size 1.45 0.45) (layers F.Cu F.Paste F.Mask) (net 33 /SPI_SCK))
  (pad 12 smd rect (at 2.95 2.275 90) (size 1.45 0.45) (layers F.Cu F.Paste F.Mask) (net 29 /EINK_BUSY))
  (pad 13 smd rect (at 2.95 1.625 90) (size 1.45 0.45) (layers F.Cu F.Paste F.Mask) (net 34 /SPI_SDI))
  (pad 14 smd rect (at 2.95 0.975 90) (size 1.45 0.45) (layers F.Cu F.Paste F.Mask) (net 40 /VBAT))
  (pad 15 smd rect (at 2.95 0.325 90) (size 1.45 0.45) (layers F.Cu F.Paste F.Mask) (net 1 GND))
  (pad 16 smd rect (at 2.95 -0.325 90) (size 1.45 0.45) (layers F.Cu F.Paste F.Mask) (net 3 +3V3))
  (pad 17 smd rect (at 2.95 -0.975 90) (size 1.45 0.45) (layers F.Cu F.Paste F.Mask) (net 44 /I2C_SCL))
  (pad 18 smd rect (at 2.95 -1.625 90) (size 1.45 0.45) (layers F.Cu F.Paste F.Mask) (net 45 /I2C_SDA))
  (pad 19 smd rect (at 2.95 -2.275 90) (size 1.45 0.45) (layers F.Cu F.Paste F.Mask) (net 35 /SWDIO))
  (pad 20 smd rect (at 2.95 -2.925 90) (size 1.45 0.45) (layers F.Cu F.Paste F.Mask) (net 37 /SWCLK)))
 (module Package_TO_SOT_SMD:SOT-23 (layer F.Cu) (at 42.545 131.445 90)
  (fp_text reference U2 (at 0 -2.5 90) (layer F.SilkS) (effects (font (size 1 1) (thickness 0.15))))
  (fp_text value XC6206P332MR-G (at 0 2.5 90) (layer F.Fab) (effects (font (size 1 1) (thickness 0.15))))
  (pad 3 smd rect (at 1 0 90) (size 0.9 0.8) (layers F.Cu F.Paste F.Mask) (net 7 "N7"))
  (pad 2 smd rect (at -1 0.95 90) (size 0.9 0.8) (layers F.Cu F.Paste F.Mask) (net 3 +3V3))
  (pad 1 smd rect (at -1 -0.95 90) (size 0.9 0.8) (layers F.Cu F.Paste F.Mask) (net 1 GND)))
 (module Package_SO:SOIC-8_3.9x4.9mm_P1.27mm (layer F.Cu) (at 29.21 137.635 270)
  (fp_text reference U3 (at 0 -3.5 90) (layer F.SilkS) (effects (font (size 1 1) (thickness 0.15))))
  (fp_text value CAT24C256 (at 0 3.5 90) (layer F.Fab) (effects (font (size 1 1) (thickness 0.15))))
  (pad 1 smd rect (at -2.7 -1.905 270) (size 1.55 0.6) (layers F.Cu F.Paste F.Mask) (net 1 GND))
  (pad 2 smd rect (at -2.7 -0.635 270) (size 1.55 0.6) (layers F.Cu F.Paste F.Mask) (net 1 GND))
  (pad 3 smd rect (at -2.7 0.635 270) (size 1.55 0.6) (layers F.Cu F.Paste F.Mask) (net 1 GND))
  (pad 4 smd rect (at -2.7 1.905 270) (size 1.55 0.6) (layers F.Cu F.Paste F.Mask) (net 1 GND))
  (pad 5 smd rect (at 2.7 1.905 270) (size 1.55 0.6) (layers F.Cu F.Paste F.Mask) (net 45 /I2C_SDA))
  (pad 6 smd rect (at 2.7 0.635 270) (size 1.55 0.6) (layers F.Cu F.Paste F.Mask) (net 44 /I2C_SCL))
  (pad 7 smd rect (at 2.7 -0.635 270) (size 1.55 0.6) (layers F.Cu F.Paste F.Mask) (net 1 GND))
  (pad 8 smd rect (at 2.7 -1.905 270) (size 1.55 0.6) (layers F.Cu F.Paste F.Mask) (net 3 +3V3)))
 (gr_line (start 63.5 118.11) (end 44.45 116.84) (layer Edge.Cuts) (width 0.05))
 (gr_arc (start 63.5 119.38) (end 64.77 119.38) (angle -90) (layer Edge.Cuts) (width 0.05))
 (gr_line (start 64.77 152.4) (end 64.77 119.38) (layer Edge.Cuts) (width 0.05))
 (gr_arc (start 63.5 152.4) (end 63.5 153.67) (angle -90) (layer Edge.Cuts) (width 0.05))
 (gr_line (start 44.45 154.94) (end 63.5 153.67) (layer Edge.Cuts) (width 0.05))
 (gr_arc (start 26.67 152.4) (end 25.4 152.4) (angle -90) (layer Edge.Cuts) (width 0.05))
 (gr_line (start 36.83 154.94) (end 26.67 153.67) (layer Edge.Cuts) (width 0.05))
 (gr_line (start 44.45 154.94) (end 36.83 154.94) (layer Edge.Cuts) (width 0.05))
 (gr_arc (start 26.67 119.38) (end 26.67 118.11) (angle -90) (layer Edge.Cuts) (width 0.05))
 (gr_line (start 36.83 116.84) (end 26.67 118.11) (layer Edge.Cuts) (width 0.05))
 (gr_line (start 44.45 116.84) (end 36.83 116.84) (layer Edge.Cuts) (width 0.05))
 (gr_line (start 25.4 119.38) (end 25.4 152.4) (layer Edge.Cuts) (width 0.05))
 (segment (start 37.886 135.89) (end 36.576 134.58) (width 0.254) (layer B.Cu) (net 2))
 (segment (start 40.64 135.89) (end 37.886 135.89) (width 0.254) (layer B.Cu) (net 2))
 (via (at 36.576 133.604) (size 0.762) (drill 0.25) (layers F.Cu B.Cu) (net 2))
 (segment (start 36.576 134.58) (end 36.576 133.604) (width 0.254) (layer B.Cu) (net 2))
 (segment (start 36.576 131.4935) (end 36.5275 131.445) (width 0.254) (layer F.Cu) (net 2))
 (segment (start 36.576 133.604) (end 36.576 131.4935) (width 0.254) (layer F.Cu) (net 2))
 (via (at 48.26 128.524) (size 0.762) (drill 0.25) (layers F.Cu B.Cu) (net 3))
 (segment (start 48.26 126.365) (end 48.26 128.524) (width 0.254) (layer F.Cu) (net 3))
 (segment (start 48.26 128.524) (end 48.26 130.55) (width 0.254) (layer F.Cu) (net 3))
 (via (at 27.559 126.238) (size 0.762) (drill 0.25) (layers F.Cu B.Cu) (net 4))
 (segment (start 26.416 126.965) (end 26.832 126.965) (width 0.254) (layer F.Cu) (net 4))
 (segment (start 26.832 126.965) (end 27.559 126.238) (width 0.254) (layer F.Cu) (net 4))
 (segment (start 27.224 126.238) (end 26.416 125.43) (width 0.254) (layer F.Cu) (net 4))
 (segment (start 27.559 126.238) (end 27.224 126.238) (width 0.254) (layer F.Cu) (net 4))
 (via (at 28.702 122.428) (size 0.762) (drill 0.25) (layers F.Cu B.Cu) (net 4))
 (segment (start 29.845 122.345) (end 28.785 122.345) (width 0.254) (layer F.Cu) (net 4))
 (segment (start 28.785 122.345) (end 28.702 122.428) (width 0.254) (layer F.Cu) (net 4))
 (segment (start 26.991 120.98) (end 26.416 120.98) (width 0.1143) (layer F.Cu) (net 19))
 (segment (start 31.7843 120.98) (end 26.991 120.98) (width 0.1143) (layer F.Cu) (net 19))
 (segment (start 32.385 121.5807) (end 31.7843 120.98) (width 0.1143) (layer F.Cu) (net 19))
 (segment (start 32.385 122.345) (end 32.385 121.5807) (width 0.1143) (layer F.Cu) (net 19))
 (segment (start 29.260049 128.600951) (end 29.260049 124.028951) (width 0.1143) (layer F.Cu) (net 20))
 (segment (start 26.416 131.445) (end 29.260049 128.600951) (width 0.1143) (layer F.Cu) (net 20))
 (segment (start 29.260049 124.028951) (end 29.845 123.444) (width 0.1143) (layer F.Cu) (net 20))
 (segment (start 31.115 122.645) (end 31.115 122.345) (width 0.1143) (layer F.Cu) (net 20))
 (segment (start 30.316 123.444) (end 31.115 122.645) (width 0.1143) (layer F.Cu) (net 20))
 (segment (start 29.845 123.444) (end 30.316 123.444) (width 0.1143) (layer F.Cu) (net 20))
 (segment (start 26.416 129.87) (end 26.416 127.935) (width 0.1143) (layer F.Cu) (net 21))
 (segment (start 26.416 122.555) (end 26.416 124.46) (width 0.1143) (layer F.Cu) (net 18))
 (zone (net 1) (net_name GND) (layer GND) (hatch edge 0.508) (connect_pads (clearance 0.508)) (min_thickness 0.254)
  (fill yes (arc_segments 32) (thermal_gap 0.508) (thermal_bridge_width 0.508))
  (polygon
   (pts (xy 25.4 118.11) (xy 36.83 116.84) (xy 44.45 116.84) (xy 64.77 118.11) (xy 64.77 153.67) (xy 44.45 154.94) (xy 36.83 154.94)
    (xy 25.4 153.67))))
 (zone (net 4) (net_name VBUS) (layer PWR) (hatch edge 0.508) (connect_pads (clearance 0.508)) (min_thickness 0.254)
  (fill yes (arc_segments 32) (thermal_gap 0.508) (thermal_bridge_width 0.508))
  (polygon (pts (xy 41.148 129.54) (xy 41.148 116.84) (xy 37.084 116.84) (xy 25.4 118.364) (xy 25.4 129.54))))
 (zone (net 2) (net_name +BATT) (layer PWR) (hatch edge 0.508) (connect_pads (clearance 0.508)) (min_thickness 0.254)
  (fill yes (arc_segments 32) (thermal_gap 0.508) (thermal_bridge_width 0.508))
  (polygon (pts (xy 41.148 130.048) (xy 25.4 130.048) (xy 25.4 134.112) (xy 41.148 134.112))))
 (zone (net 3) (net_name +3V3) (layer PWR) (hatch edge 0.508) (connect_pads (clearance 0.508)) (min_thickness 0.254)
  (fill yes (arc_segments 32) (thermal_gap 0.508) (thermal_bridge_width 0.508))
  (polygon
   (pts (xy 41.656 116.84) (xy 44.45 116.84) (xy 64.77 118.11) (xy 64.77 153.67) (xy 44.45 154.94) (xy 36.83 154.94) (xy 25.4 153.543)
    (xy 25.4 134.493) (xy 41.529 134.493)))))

